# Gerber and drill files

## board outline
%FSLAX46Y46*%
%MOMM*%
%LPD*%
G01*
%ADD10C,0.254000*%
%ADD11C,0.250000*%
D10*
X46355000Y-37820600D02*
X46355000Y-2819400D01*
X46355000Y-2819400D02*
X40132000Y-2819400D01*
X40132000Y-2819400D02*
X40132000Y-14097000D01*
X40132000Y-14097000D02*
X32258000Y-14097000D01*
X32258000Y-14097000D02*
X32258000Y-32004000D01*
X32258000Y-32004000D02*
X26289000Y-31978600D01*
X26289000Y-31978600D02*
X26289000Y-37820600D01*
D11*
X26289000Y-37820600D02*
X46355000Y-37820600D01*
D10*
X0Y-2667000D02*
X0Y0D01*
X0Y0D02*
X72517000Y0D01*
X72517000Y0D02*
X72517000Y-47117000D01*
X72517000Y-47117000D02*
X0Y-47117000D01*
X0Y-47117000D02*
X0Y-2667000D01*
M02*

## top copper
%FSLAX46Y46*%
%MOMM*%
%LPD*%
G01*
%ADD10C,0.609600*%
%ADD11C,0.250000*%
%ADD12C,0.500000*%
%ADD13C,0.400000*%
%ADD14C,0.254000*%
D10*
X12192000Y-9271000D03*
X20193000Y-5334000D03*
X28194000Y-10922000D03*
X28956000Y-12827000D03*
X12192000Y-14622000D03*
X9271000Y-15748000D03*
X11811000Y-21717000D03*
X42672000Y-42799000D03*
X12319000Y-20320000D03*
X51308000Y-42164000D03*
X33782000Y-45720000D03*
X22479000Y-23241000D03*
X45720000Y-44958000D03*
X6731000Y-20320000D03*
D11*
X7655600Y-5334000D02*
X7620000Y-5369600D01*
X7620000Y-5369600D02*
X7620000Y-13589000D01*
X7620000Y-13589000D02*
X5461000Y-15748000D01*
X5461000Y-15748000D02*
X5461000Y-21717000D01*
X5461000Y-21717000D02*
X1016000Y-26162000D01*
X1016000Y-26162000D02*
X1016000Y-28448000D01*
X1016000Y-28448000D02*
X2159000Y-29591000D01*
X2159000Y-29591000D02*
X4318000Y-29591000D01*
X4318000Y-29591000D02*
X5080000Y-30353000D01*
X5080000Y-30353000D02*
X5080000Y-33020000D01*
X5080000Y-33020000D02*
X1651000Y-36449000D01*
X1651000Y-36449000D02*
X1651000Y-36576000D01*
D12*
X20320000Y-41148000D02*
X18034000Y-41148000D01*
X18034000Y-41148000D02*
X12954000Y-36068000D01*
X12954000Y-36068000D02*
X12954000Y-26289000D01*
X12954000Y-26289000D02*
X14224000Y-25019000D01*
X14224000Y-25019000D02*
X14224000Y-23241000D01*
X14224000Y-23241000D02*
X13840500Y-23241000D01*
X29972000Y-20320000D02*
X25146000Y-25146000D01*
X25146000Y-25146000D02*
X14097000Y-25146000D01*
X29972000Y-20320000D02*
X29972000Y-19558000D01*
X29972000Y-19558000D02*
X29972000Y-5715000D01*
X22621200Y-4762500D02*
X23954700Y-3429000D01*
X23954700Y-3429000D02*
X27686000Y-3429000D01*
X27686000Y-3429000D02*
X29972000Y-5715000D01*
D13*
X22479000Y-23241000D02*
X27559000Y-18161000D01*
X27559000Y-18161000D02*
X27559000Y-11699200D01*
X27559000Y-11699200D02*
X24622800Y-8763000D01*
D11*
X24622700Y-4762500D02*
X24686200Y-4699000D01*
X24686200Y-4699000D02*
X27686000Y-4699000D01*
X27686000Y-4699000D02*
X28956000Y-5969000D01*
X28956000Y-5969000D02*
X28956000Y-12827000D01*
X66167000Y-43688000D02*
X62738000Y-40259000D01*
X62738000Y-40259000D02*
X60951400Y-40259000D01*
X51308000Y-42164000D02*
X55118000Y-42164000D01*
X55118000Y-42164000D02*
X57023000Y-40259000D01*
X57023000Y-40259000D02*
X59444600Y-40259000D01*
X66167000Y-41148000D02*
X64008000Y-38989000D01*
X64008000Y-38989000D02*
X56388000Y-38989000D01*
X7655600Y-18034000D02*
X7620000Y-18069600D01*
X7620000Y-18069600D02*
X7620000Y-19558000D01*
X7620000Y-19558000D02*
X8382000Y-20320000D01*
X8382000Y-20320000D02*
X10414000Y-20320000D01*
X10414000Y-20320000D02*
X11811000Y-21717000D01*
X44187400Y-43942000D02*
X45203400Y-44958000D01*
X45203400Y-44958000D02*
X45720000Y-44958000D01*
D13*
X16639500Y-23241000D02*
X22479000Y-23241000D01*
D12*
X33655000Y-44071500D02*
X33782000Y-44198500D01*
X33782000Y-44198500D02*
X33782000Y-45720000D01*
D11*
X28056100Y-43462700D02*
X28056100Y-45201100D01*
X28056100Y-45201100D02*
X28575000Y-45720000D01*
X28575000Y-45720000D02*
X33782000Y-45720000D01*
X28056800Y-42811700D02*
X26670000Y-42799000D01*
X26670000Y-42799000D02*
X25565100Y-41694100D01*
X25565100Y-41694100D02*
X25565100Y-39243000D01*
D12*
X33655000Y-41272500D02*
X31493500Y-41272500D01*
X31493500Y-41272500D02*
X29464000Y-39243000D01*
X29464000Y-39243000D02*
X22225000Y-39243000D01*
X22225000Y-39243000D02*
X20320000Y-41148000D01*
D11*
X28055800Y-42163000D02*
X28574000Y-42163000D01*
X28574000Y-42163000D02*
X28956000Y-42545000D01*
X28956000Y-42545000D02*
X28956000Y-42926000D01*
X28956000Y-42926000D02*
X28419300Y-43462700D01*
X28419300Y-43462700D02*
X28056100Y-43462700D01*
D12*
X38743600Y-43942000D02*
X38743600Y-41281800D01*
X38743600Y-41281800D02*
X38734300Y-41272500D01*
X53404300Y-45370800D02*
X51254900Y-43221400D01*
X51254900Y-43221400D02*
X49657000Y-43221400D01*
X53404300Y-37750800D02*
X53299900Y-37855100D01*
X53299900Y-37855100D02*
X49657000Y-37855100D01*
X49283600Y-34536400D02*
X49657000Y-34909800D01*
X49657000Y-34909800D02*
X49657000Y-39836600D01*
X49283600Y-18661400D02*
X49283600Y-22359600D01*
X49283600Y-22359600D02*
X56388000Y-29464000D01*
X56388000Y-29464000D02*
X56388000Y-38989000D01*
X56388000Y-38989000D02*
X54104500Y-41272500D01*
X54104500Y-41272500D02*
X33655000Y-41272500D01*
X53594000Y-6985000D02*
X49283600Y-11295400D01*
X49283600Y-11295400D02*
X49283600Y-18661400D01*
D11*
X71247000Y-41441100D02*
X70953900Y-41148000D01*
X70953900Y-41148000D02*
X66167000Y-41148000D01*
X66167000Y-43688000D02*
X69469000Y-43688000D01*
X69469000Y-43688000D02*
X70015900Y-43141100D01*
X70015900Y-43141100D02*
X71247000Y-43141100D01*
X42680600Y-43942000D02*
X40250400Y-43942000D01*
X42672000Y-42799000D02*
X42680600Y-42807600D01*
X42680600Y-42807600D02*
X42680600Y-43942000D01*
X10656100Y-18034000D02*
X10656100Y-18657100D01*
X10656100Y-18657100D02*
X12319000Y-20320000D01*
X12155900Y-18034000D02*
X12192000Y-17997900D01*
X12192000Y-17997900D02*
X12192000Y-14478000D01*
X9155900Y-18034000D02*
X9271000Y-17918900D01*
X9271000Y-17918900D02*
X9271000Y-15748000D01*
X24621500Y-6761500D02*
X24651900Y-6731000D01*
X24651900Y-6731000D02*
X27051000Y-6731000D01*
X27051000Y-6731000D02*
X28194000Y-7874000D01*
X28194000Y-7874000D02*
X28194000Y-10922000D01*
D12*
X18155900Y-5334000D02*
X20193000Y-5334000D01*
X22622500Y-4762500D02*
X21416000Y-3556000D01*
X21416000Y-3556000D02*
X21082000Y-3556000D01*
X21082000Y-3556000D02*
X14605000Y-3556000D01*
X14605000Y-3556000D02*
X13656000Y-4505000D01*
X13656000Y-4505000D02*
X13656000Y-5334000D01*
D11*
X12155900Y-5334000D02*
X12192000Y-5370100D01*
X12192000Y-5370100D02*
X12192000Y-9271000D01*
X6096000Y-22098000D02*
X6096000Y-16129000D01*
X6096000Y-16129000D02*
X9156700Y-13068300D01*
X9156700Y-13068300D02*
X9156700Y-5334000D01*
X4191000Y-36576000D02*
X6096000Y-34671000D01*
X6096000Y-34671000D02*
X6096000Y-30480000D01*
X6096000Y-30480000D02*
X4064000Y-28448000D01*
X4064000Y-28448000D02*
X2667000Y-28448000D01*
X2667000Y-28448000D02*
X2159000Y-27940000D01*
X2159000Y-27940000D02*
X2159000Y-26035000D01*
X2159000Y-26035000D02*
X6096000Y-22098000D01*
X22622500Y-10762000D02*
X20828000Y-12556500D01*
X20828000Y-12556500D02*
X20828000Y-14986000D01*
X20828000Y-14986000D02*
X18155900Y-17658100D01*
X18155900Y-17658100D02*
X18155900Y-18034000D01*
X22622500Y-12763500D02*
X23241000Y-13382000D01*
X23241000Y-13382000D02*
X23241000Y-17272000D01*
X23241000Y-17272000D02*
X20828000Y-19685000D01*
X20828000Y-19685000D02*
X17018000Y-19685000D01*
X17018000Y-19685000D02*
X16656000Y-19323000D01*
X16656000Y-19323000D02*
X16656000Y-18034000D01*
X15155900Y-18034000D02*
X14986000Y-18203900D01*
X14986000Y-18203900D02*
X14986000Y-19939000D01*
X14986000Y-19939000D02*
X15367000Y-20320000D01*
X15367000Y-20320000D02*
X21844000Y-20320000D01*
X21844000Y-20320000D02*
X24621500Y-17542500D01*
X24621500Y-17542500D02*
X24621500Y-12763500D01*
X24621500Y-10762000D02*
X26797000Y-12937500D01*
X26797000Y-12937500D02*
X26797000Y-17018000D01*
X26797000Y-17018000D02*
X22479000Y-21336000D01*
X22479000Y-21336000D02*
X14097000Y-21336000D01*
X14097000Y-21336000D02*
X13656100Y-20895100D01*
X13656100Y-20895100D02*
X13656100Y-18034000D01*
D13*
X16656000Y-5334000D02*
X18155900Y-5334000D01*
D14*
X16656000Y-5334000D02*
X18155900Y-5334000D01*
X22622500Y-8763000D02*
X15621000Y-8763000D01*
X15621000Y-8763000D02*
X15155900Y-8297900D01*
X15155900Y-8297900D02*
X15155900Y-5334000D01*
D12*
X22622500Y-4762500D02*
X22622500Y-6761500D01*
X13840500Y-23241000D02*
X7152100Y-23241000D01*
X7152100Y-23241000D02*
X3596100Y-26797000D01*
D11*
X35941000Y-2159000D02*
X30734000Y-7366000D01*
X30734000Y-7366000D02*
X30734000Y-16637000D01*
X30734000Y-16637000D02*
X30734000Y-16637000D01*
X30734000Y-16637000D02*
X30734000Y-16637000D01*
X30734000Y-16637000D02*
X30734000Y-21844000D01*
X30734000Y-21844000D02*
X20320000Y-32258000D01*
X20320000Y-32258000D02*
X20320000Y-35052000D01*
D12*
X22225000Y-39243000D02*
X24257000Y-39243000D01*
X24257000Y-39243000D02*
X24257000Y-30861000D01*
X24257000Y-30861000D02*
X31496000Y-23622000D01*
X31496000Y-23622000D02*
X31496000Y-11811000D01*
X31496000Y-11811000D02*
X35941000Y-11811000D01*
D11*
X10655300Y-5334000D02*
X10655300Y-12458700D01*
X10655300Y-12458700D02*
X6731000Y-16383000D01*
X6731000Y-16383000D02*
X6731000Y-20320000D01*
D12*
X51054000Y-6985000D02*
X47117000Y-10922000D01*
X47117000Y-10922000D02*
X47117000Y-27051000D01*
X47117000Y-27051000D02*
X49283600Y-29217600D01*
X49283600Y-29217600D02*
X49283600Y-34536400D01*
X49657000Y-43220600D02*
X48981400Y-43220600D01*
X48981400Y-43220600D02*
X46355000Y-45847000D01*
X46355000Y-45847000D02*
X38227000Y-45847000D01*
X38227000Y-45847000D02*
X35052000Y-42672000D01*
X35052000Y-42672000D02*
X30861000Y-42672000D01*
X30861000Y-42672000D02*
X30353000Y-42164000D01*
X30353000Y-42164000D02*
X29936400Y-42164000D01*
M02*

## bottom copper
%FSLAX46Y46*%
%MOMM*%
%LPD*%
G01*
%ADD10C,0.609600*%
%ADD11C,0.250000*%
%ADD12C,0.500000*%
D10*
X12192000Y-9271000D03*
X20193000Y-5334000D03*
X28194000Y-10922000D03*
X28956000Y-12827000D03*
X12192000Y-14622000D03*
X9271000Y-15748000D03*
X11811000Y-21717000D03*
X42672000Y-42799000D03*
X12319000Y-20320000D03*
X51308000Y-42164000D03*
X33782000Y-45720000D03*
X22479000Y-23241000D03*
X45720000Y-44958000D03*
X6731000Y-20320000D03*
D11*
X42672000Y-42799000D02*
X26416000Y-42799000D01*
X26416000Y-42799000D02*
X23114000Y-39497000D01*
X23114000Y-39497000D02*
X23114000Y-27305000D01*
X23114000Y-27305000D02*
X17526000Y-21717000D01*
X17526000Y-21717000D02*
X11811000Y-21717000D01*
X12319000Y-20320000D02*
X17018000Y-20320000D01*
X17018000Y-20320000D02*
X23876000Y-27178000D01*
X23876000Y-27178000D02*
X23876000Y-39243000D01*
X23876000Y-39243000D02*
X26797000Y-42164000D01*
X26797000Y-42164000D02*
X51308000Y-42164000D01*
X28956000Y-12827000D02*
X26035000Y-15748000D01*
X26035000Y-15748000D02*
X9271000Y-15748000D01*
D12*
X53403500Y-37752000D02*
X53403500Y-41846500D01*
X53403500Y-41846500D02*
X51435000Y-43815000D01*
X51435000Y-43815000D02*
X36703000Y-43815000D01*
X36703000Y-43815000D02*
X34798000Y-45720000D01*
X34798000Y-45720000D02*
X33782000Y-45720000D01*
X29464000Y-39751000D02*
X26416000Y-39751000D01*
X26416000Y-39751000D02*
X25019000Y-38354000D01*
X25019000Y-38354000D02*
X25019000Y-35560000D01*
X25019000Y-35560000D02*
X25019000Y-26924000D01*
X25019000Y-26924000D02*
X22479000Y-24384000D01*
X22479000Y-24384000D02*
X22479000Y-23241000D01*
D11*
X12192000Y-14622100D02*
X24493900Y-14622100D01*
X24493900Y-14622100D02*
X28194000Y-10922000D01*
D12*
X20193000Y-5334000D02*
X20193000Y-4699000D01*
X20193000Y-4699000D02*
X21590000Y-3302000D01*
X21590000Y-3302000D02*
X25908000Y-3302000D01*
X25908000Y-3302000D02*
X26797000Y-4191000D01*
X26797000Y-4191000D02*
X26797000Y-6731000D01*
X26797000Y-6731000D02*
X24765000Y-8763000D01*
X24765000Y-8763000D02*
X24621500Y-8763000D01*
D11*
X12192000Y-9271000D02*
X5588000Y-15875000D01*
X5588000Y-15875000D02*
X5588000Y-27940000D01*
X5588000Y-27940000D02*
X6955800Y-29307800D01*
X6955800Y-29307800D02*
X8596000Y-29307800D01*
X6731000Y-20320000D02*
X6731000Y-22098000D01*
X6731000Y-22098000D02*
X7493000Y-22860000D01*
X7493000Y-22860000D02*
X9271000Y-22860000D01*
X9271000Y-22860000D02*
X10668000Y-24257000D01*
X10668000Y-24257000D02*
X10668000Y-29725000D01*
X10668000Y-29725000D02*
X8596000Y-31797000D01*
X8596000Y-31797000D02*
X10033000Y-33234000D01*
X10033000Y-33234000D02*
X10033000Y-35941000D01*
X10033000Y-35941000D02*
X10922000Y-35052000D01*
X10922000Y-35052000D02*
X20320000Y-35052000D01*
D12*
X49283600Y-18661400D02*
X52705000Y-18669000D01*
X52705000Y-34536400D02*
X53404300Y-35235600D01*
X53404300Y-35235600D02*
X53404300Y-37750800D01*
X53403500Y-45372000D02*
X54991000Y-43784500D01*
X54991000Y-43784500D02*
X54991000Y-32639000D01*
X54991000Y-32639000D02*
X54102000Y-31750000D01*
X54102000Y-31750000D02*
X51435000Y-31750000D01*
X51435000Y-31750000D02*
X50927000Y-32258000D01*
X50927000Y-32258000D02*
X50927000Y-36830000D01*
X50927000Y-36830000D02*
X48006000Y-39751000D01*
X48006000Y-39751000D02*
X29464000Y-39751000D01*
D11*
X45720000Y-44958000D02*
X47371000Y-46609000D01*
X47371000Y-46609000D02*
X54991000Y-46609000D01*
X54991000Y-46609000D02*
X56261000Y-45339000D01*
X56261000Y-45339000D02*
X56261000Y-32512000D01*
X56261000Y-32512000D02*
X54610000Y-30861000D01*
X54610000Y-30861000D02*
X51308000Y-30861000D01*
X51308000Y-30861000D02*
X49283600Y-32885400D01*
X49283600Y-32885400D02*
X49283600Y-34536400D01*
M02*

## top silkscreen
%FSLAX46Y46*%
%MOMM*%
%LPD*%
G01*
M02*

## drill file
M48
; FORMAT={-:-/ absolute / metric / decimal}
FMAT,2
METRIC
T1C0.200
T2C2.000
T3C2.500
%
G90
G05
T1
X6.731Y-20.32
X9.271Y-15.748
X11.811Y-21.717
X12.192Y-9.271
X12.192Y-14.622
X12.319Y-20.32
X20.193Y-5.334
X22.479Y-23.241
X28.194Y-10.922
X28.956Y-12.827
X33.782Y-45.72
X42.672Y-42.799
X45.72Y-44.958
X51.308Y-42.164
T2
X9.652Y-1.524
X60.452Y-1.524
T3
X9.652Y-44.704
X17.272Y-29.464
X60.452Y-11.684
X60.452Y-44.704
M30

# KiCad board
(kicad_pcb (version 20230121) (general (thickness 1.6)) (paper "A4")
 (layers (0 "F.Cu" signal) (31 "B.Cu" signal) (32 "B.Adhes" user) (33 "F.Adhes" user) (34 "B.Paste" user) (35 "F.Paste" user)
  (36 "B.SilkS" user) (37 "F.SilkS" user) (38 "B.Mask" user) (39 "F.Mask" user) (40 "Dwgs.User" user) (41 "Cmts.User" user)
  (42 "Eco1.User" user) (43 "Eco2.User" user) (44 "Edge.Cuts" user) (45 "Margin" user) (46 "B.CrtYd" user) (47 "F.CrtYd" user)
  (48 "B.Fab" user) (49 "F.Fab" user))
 (gr_line (start 46.3550 37.8206) (end 46.3550 2.8194) (layer "Edge.Cuts") (width 0.2540))
 (gr_line (start 46.3550 2.8194) (end 40.1320 2.8194) (layer "Edge.Cuts") (width 0.2540))
 (gr_line (start 40.1320 2.8194) (end 40.1320 14.0970) (layer "Edge.Cuts") (width 0.2540))
 (gr_line (start 40.1320 14.0970) (end 32.2580 14.0970) (layer "Edge.Cuts") (width 0.2540))
 (gr_line (start 32.2580 14.0970) (end 32.2580 32.0040) (layer "Edge.Cuts") (width 0.2540))
 (gr_line (start 32.2580 32.0040) (end 26.2890 31.9786) (layer "Edge.Cuts") (width 0.2540))
 (gr_line (start 26.2890 31.9786) (end 26.2890 37.8206) (layer "Edge.Cuts") (width 0.2540))
 (gr_line (start 26.2890 37.8206) (end 46.3550 37.8206) (layer "Edge.Cuts") (width 0.2500))
 (gr_line (start 0.0000 2.6670) (end 0.0000 0.0000) (layer "Edge.Cuts") (width 0.2540))
 (gr_line (start 0.0000 0.0000) (end 72.5170 0.0000) (layer "Edge.Cuts") (width 0.2540))
 (gr_line (start 72.5170 0.0000) (end 72.5170 47.1170) (layer "Edge.Cuts") (width 0.2540))
 (gr_line (start 72.5170 47.1170) (end 0.0000 47.1170) (layer "Edge.Cuts") (width 0.2540))
 (gr_line (start 0.0000 47.1170) (end 0.0000 2.6670) (layer "Edge.Cuts") (width 0.2540))
 (segment (start 7.6556 5.3340) (end 7.6200 5.3696) (width 0.2500) (layer "F.Cu") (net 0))
 (segment (start 7.6200 5.3696) (end 7.6200 13.5890) (width 0.2500) (layer "F.Cu") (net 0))
 (segment (start 7.6200 13.5890) (end 5.4610 15.7480) (width 0.2500) (layer "F.Cu") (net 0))
 (segment (start 5.4610 15.7480) (end 5.4610 21.7170) (width 0.2500) (layer "F.Cu") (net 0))
 (segment (start 5.4610 21.7170) (end 1.0160 26.1620) (width 0.2500) (layer "F.Cu") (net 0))
 (segment (start 1.0160 26.1620) (end 1.0160 28.4480) (width 0.2500) (layer "F.Cu") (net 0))
 (segment (start 1.0160 28.4480) (end 2.1590 29.5910) (width 0.2500) (layer "F.Cu") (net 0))
 (segment (start 2.1590 29.5910) (end 4.3180 29.5910) (width 0.2500) (layer "F.Cu") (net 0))
 (segment (start 4.3180 29.5910) (end 5.0800 30.3530) (width 0.2500) (layer "F.Cu") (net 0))
 (segment (start 5.0800 30.3530) (end 5.0800 33.0200) (width 0.2500) (layer "F.Cu") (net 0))
 (segment (start 5.0800 33.0200) (end 1.6510 36.4490) (width 0.2500) (layer "F.Cu") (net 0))
 (segment (start 1.6510 36.4490) (end 1.6510 36.5760) (width 0.2500) (layer "F.Cu") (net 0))
 (segment (start 20.3200 41.1480) (end 18.0340 41.1480) (width 0.5000) (layer "F.Cu") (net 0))
 (segment (start 18.0340 41.1480) (end 12.9540 36.0680) (width 0.5000) (layer "F.Cu") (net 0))
 (segment (start 12.9540 36.0680) (end 12.9540 26.2890) (width 0.5000) (layer "F.Cu") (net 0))
 (segment (start 12.9540 26.2890) (end 14.2240 25.0190) (width 0.5000) (layer "F.Cu") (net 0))
 (segment (start 14.2240 25.0190) (end 14.2240 23.2410) (width 0.5000) (layer "F.Cu") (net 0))
 (segment (start 14.2240 23.2410) (end 13.8405 23.2410) (width 0.5000) (layer "F.Cu") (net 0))
 (segment (start 29.9720 20.3200) (end 25.1460 25.1460) (width 0.5000) (layer "F.Cu") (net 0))
 (segment (start 25.1460 25.1460) (end 14.0970 25.1460) (width 0.5000) (layer "F.Cu") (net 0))
 (segment (start 29.9720 20.3200) (end 29.9720 19.5580) (width 0.5000) (layer "F.Cu") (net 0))
 (segment (start 29.9720 19.5580) (end 29.9720 5.7150) (width 0.5000) (layer "F.Cu") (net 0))
 (segment (start 22.6212 4.7625) (end 23.9547 3.4290) (width 0.5000) (layer "F.Cu") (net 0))
 (segment (start 23.9547 3.4290) (end 27.6860 3.4290) (width 0.5000) (layer "F.Cu") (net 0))
 (segment (start 27.6860 3.4290) (end 29.9720 5.7150) (width 0.5000) (layer "F.Cu") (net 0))
 (segment (start 22.4790 23.2410) (end 27.5590 18.1610) (width 0.4000) (layer "F.Cu") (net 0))
 (segment (start 27.5590 18.1610) (end 27.5590 11.6992) (width 0.4000) (layer "F.Cu") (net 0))
 (segment (start 27.5590 11.6992) (end 24.6228 8.7630) (width 0.4000) (layer "F.Cu") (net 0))
 (segment (start 24.6227 4.7625) (end 24.6862 4.6990) (width 0.2500) (layer "F.Cu") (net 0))
 (segment (start 24.6862 4.6990) (end 27.6860 4.6990) (width 0.2500) (layer "F.Cu") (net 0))
 (segment (start 27.6860 4.6990) (end 28.9560 5.9690) (width 0.2500) (layer "F.Cu") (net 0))
 (segment (start 28.9560 5.9690) (end 28.9560 12.8270) (width 0.2500) (layer "F.Cu") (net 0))
 (segment (start 66.1670 43.6880) (end 62.7380 40.2590) (width 0.2500) (layer "F.Cu") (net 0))
 (segment (start 62.7380 40.2590) (end 60.9514 40.2590) (width 0.2500) (layer "F.Cu") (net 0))
 (segment (start 51.3080 42.1640) (end 55.1180 42.1640) (width 0.2500) (layer "F.Cu") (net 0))
 (segment (start 55.1180 42.1640) (end 57.0230 40.2590) (width 0.2500) (layer "F.Cu") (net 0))
 (segment (start 57.0230 40.2590) (end 59.4446 40.2590) (width 0.2500) (layer "F.Cu") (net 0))
 (segment (start 66.1670 41.1480) (end 64.0080 38.9890) (width 0.2500) (layer "F.Cu") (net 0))
 (segment (start 64.0080 38.9890) (end 56.3880 38.9890) (width 0.2500) (layer "F.Cu") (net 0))
 (segment (start 7.6556 18.0340) (end 7.6200 18.0696) (width 0.2500) (layer "F.Cu") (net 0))
 (segment (start 7.6200 18.0696) (end 7.6200 19.5580) (width 0.2500) (layer "F.Cu") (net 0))
 (segment (start 7.6200 19.5580) (end 8.3820 20.3200) (width 0.2500) (layer "F.Cu") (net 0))
 (segment (start 8.3820 20.3200) (end 10.4140 20.3200) (width 0.2500) (layer "F.Cu") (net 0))
 (segment (start 10.4140 20.3200) (end 11.8110 21.7170) (width 0.2500) (layer "F.Cu") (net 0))
 (segment (start 44.1874 43.9420) (end 45.2034 44.9580) (width 0.2500) (layer "F.Cu") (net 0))
 (segment (start 45.2034 44.9580) (end 45.7200 44.9580) (width 0.2500) (layer "F.Cu") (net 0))
 (segment (start 16.6395 23.2410) (end 22.4790 23.2410) (width 0.4000) (layer "F.Cu") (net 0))
 (segment (start 33.6550 44.0715) (end 33.7820 44.1985) (width 0.5000) (layer "F.Cu") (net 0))
 (segment (start 33.7820 44.1985) (end 33.7820 45.7200) (width 0.5000) (layer "F.Cu") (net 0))
 (segment (start 28.0561 43.4627) (end 28.0561 45.2011) (width 0.2500) (layer "F.Cu") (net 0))
 (segment (start 28.0561 45.2011) (end 28.5750 45.7200) (width 0.2500) (layer "F.Cu") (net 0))
 (segment (start 28.5750 45.7200) (end 33.7820 45.7200) (width 0.2500) (layer "F.Cu") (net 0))
 (segment (start 28.0568 42.8117) (end 26.6700 42.7990) (width 0.2500) (layer "F.Cu") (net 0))
 (segment (start 26.6700 42.7990) (end 25.5651 41.6941) (width 0.2500) (layer "F.Cu") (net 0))
 (segment (start 25.5651 41.6941) (end 25.5651 39.2430) (width 0.2500) (layer "F.Cu") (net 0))
 (segment (start 33.6550 41.2725) (end 31.4935 41.2725) (width 0.5000) (layer "F.Cu") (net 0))
 (segment (start 31.4935 41.2725) (end 29.4640 39.2430) (width 0.5000) (layer "F.Cu") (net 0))
 (segment (start 29.4640 39.2430) (end 22.2250 39.2430) (width 0.5000) (layer "F.Cu") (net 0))
 (segment (start 22.2250 39.2430) (end 20.3200 41.1480) (width 0.5000) (layer "F.Cu") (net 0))
 (segment (start 28.0558 42.1630) (end 28.5740 42.1630) (width 0.2500) (layer "F.Cu") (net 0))
 (segment (start 28.5740 42.1630) (end 28.9560 42.5450) (width 0.2500) (layer "F.Cu") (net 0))
 (segment (start 28.9560 42.5450) (end 28.9560 42.9260) (width 0.2500) (layer "F.Cu") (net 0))
 (segment (start 28.9560 42.9260) (end 28.4193 43.4627) (width 0.2500) (layer "F.Cu") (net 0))
 (segment (start 28.4193 43.4627) (end 28.0561 43.4627) (width 0.2500) (layer "F.Cu") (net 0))
 (segment (start 38.7436 43.9420) (end 38.7436 41.2818) (width 0.5000) (layer "F.Cu") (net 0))
 (segment (start 38.7436 41.2818) (end 38.7343 41.2725) (width 0.5000) (layer "F.Cu") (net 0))
 (segment (start 53.4043 45.3708) (end 51.2549 43.2214) (width 0.5000) (layer "F.Cu") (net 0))
 (segment (start 51.2549 43.2214) (end 49.6570 43.2214) (width 0.5000) (layer "F.Cu") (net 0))
 (segment (start 53.4043 37.7508) (end 53.2999 37.8551) (width 0.5000) (layer "F.Cu") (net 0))
 (segment (start 53.2999 37.8551) (end 49.6570 37.8551) (width 0.5000) (layer "F.Cu") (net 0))
 (segment (start 49.2836 34.5364) (end 49.6570 34.9098) (width 0.5000) (layer "F.Cu") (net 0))
 (segment (start 49.6570 34.9098) (end 49.6570 39.8366) (width 0.5000) (layer "F.Cu") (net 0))
 (segment (start 49.2836 18.6614) (end 49.2836 22.3596) (width 0.5000) (layer "F.Cu") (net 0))
 (segment (start 49.2836 22.3596) (end 56.3880 29.4640) (width 0.5000) (layer "F.Cu") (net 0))
 (segment (start 56.3880 29.4640) (end 56.3880 38.9890) (width 0.5000) (layer "F.Cu") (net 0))
 (segment (start 56.3880 38.9890) (end 54.1045 41.2725) (width 0.5000) (layer "F.Cu") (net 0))
 (segment (start 54.1045 41.2725) (end 33.6550 41.2725) (width 0.5000) (layer "F.Cu") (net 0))
 (segment (start 53.5940 6.9850) (end 49.2836 11.2954) (width 0.5000) (layer "F.Cu") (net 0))
 (segment (start 49.2836 11.2954) (end 49.2836 18.6614) (width 0.5000) (layer "F.Cu") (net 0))
 (segment (start 71.2470 41.4411) (end 70.9539 41.1480) (width 0.2500) (layer "F.Cu") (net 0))
 (segment (start 70.9539 41.1480) (end 66.1670 41.1480) (width 0.2500) (layer "F.Cu") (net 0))
 (segment (start 66.1670 43.6880) (end 69.4690 43.6880) (width 0.2500) (layer "F.Cu") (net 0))
 (segment (start 69.4690 43.6880) (end 70.0159 43.1411) (width 0.2500) (layer "F.Cu") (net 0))
 (segment (start 70.0159 43.1411) (end 71.2470 43.1411) (width 0.2500) (layer "F.Cu") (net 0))
 (segment (start 42.6806 43.9420) (end 40.2504 43.9420) (width 0.2500) (layer "F.Cu") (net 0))
 (segment (start 42.6720 42.7990) (end 42.6806 42.8076) (width 0.2500) (layer "F.Cu") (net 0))
 (segment (start 42.6806 42.8076) (end 42.6806 43.9420) (width 0.2500) (layer "F.Cu") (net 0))
 (segment (start 10.6561 18.0340) (end 10.6561 18.6571) (width 0.2500) (layer "F.Cu") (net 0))
 (segment (start 10.6561 18.6571) (end 12.3190 20.3200) (width 0.2500) (layer "F.Cu") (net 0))
 (segment (start 12.1559 18.0340) (end 12.1920 17.9979) (width 0.2500) (layer "F.Cu") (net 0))
 (segment (start 12.1920 17.9979) (end 12.1920 14.4780) (width 0.2500) (layer "F.Cu") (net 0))
 (segment (start 9.1559 18.0340) (end 9.2710 17.9189) (width 0.2500) (layer "F.Cu") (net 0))
 (segment (start 9.2710 17.9189) (end 9.2710 15.7480) (width 0.2500) (layer "F.Cu") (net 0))
 (segment (start 24.6215 6.7615) (end 24.6519 6.7310) (width 0.2500) (layer "F.Cu") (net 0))
 (segment (start 24.6519 6.7310) (end 27.0510 6.7310) (width 0.2500) (layer "F.Cu") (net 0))
 (segment (start 27.0510 6.7310) (end 28.1940 7.8740) (width 0.2500) (layer "F.Cu") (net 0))
 (segment (start 28.1940 7.8740) (end 28.1940 10.9220) (width 0.2500) (layer "F.Cu") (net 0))
 (segment (start 18.1559 5.3340) (end 20.1930 5.3340) (width 0.5000) (layer "F.Cu") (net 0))
 (segment (start 22.6225 4.7625) (end 21.4160 3.5560) (width 0.5000) (layer "F.Cu") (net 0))
 (segment (start 21.4160 3.5560) (end 21.0820 3.5560) (width 0.5000) (layer "F.Cu") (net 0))
 (segment (start 21.0820 3.5560) (end 14.6050 3.5560) (width 0.5000) (layer "F.Cu") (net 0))
 (segment (start 14.6050 3.5560) (end 13.6560 4.5050) (width 0.5000) (layer "F.Cu") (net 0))
 (segment (start 13.6560 4.5050) (end 13.6560 5.3340) (width 0.5000) (layer "F.Cu") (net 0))
 (segment (start 12.1559 5.3340) (end 12.1920 5.3701) (width 0.2500) (layer "F.Cu") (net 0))
 (segment (start 12.1920 5.3701) (end 12.1920 9.2710) (width 0.2500) (layer "F.Cu") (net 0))
 (segment (start 6.0960 22.0980) (end 6.0960 16.1290) (width 0.2500) (layer "F.Cu") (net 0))
 (segment (start 6.0960 16.1290) (end 9.1567 13.0683) (width 0.2500) (layer "F.Cu") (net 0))
 (segment (start 9.1567 13.0683) (end 9.1567 5.3340) (width 0.2500) (layer "F.Cu") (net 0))
 (segment (start 4.1910 36.5760) (end 6.0960 34.6710) (width 0.2500) (layer "F.Cu") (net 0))
 (segment (start 6.0960 34.6710) (end 6.0960 30.4800) (width 0.2500) (layer "F.Cu") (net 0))
 (segment (start 6.0960 30.4800) (end 4.0640 28.4480) (width 0.2500) (layer "F.Cu") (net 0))
 (segment (start 4.0640 28.4480) (end 2.6670 28.4480) (width 0.2500) (layer "F.Cu") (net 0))
 (segment (start 2.6670 28.4480) (end 2.1590 27.9400) (width 0.2500) (layer "F.Cu") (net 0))
 (segment (start 2.1590 27.9400) (end 2.1590 26.0350) (width 0.2500) (layer "F.Cu") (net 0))
 (segment (start 2.1590 26.0350) (end 6.0960 22.0980) (width 0.2500) (layer "F.Cu") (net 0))
 (segment (start 22.6225 10.7620) (end 20.8280 12.5565) (width 0.2500) (layer "F.Cu") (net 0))
 (segment (start 20.8280 12.5565) (end 20.8280 14.9860) (width 0.2500) (layer "F.Cu") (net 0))
 (segment (start 20.8280 14.9860) (end 18.1559 17.6581) (width 0.2500) (layer "F.Cu") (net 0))
 (segment (start 18.1559 17.6581) (end 18.1559 18.0340) (width 0.2500) (layer "F.Cu") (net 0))
 (segment (start 22.6225 12.7635) (end 23.2410 13.3820) (width 0.2500) (layer "F.Cu") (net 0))
 (segment (start 23.2410 13.3820) (end 23.2410 17.2720) (width 0.2500) (layer "F.Cu") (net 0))
 (segment (start 23.2410 17.2720) (end 20.8280 19.6850) (width 0.2500) (layer "F.Cu") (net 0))
 (segment (start 20.8280 19.6850) (end 17.0180 19.6850) (width 0.2500) (layer "F.Cu") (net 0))
 (segment (start 17.0180 19.6850) (end 16.6560 19.3230) (width 0.2500) (layer "F.Cu") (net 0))
 (segment (start 16.6560 19.3230) (end 16.6560 18.0340) (width 0.2500) (layer "F.Cu") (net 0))
 (segment (start 15.1559 18.0340) (end 14.9860 18.2039) (width 0.2500) (layer "F.Cu") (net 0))
 (segment (start 14.9860 18.2039) (end 14.9860 19.9390) (width 0.2500) (layer "F.Cu") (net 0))
 (segment (start 14.9860 19.9390) (end 15.3670 20.3200) (width 0.2500) (layer "F.Cu") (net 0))
 (segment (start 15.3670 20.3200) (end 21.8440 20.3200) (width 0.2500) (layer "F.Cu") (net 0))
 (segment (start 21.8440 20.3200) (end 24.6215 17.5425) (width 0.2500) (layer "F.Cu") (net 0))
 (segment (start 24.6215 17.5425) (end 24.6215 12.7635) (width 0.2500) (layer "F.Cu") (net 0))
 (segment (start 24.6215 10.7620) (end 26.7970 12.9375) (width 0.2500) (layer "F.Cu") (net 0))
 (segment (start 26.7970 12.9375) (end 26.7970 17.0180) (width 0.2500) (layer "F.Cu") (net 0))
 (segment (start 26.7970 17.0180) (end 22.4790 21.3360) (width 0.2500) (layer "F.Cu") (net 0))
 (segment (start 22.4790 21.3360) (end 14.0970 21.3360) (width 0.2500) (layer "F.Cu") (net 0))
 (segment (start 14.0970 21.3360) (end 13.6561 20.8951) (width 0.2500) (layer "F.Cu") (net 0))
 (segment (start 13.6561 20.8951) (end 13.6561 18.0340) (width 0.2500) (layer "F.Cu") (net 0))
 (segment (start 16.6560 5.3340) (end 18.1559 5.3340) (width 0.4000) (layer "F.Cu") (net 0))
 (segment (start 16.6560 5.3340) (end 18.1559 5.3340) (width 0.2540) (layer "F.Cu") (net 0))
 (segment (start 22.6225 8.7630) (end 15.6210 8.7630) (width 0.2540) (layer "F.Cu") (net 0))
 (segment (start 15.6210 8.7630) (end 15.1559 8.2979) (width 0.2540) (layer "F.Cu") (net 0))
 (segment (start 15.1559 8.2979) (end 15.1559 5.3340) (width 0.2540) (layer "F.Cu") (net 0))
 (segment (start 22.6225 4.7625) (end 22.6225 6.7615) (width 0.5000) (layer "F.Cu") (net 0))
 (segment (start 13.8405 23.2410) (end 7.1521 23.2410) (width 0.5000) (layer "F.Cu") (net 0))
 (segment (start 7.1521 23.2410) (end 3.5961 26.7970) (width 0.5000) (layer "F.Cu") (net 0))
 (segment (start 35.9410 2.1590) (end 30.7340 7.3660) (width 0.2500) (layer "F.Cu") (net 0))
 (segment (start 30.7340 7.3660) (end 30.7340 16.6370) (width 0.2500) (layer "F.Cu") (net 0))
 (segment (start 30.7340 16.6370) (end 30.7340 16.6370) (width 0.2500) (layer "F.Cu") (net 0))
 (segment (start 30.7340 16.6370) (end 30.7340 16.6370) (width 0.2500) (layer "F.Cu") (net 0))
 (segment (start 30.7340 16.6370) (end 30.7340 21.8440) (width 0.2500) (layer "F.Cu") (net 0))
 (segment (start 30.7340 21.8440) (end 20.3200 32.2580) (width 0.2500) (layer "F.Cu") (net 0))
 (segment (start 20.3200 32.2580) (end 20.3200 35.0520) (width 0.2500) (layer "F.Cu") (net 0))
 (segment (start 22.2250 39.2430) (end 24.2570 39.2430) (width 0.5000) (layer "F.Cu") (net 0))
 (segment (start 24.2570 39.2430) (end 24.2570 30.8610) (width 0.5000) (layer "F.Cu") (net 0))
 (segment (start 24.2570 30.8610) (end 31.4960 23.6220) (width 0.5000) (layer "F.Cu") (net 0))
 (segment (start 31.4960 23.6220) (end 31.4960 11.8110) (width 0.5000) (layer "F.Cu") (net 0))
 (segment (start 31.4960 11.8110) (end 35.9410 11.8110) (width 0.5000) (layer "F.Cu") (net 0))
 (segment (start 10.6553 5.3340) (end 10.6553 12.4587) (width 0.2500) (layer "F.Cu") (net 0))
 (segment (start 10.6553 12.4587) (end 6.7310 16.3830) (width 0.2500) (layer "F.Cu") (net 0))
 (segment (start 6.7310 16.3830) (end 6.7310 20.3200) (width 0.2500) (layer "F.Cu") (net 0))
 (segment (start 51.0540 6.9850) (end 47.1170 10.9220) (width 0.5000) (layer "F.Cu") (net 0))
 (segment (start 47.1170 10.9220) (end 47.1170 27.0510) (width 0.5000) (layer "F.Cu") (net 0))
 (segment (start 47.1170 27.0510) (end 49.2836 29.2176) (width 0.5000) (layer "F.Cu") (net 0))
 (segment (start 49.2836 29.2176) (end 49.2836 34.5364) (width 0.5000) (layer "F.Cu") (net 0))
 (segment (start 49.6570 43.2206) (end 48.9814 43.2206) (width 0.5000) (layer "F.Cu") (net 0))
 (segment (start 48.9814 43.2206) (end 46.3550 45.8470) (width 0.5000) (layer "F.Cu") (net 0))
 (segment (start 46.3550 45.8470) (end 38.2270 45.8470) (width 0.5000) (layer "F.Cu") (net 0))
 (segment (start 38.2270 45.8470) (end 35.0520 42.6720) (width 0.5000) (layer "F.Cu") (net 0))
 (segment (start 35.0520 42.6720) (end 30.8610 42.6720) (width 0.5000) (layer "F.Cu") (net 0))
 (segment (start 30.8610 42.6720) (end 30.3530 42.1640) (width 0.5000) (layer "F.Cu") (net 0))
 (segment (start 30.3530 42.1640) (end 29.9364 42.1640) (width 0.5000) (layer "F.Cu") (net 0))
 (segment (start 42.6720 42.7990) (end 26.4160 42.7990) (width 0.2500) (layer "B.Cu") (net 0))
 (segment (start 26.4160 42.7990) (end 23.1140 39.4970) (width 0.2500) (layer "B.Cu") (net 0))
 (segment (start 23.1140 39.4970) (end 23.1140 27.3050) (width 0.2500) (layer "B.Cu") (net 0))
 (segment (start 23.1140 27.3050) (end 17.5260 21.7170) (width 0.2500) (layer "B.Cu") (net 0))
 (segment (start 17.5260 21.7170) (end 11.8110 21.7170) (width 0.2500) (layer "B.Cu") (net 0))
 (segment (start 12.3190 20.3200) (end 17.0180 20.3200) (width 0.2500) (layer "B.Cu") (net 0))
 (segment (start 17.0180 20.3200) (end 23.8760 27.1780) (width 0.2500) (layer "B.Cu") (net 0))
 (segment (start 23.8760 27.1780) (end 23.8760 39.2430) (width 0.2500) (layer "B.Cu") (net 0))
 (segment (start 23.8760 39.2430) (end 26.7970 42.1640) (width 0.2500) (layer "B.Cu") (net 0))
 (segment (start 26.7970 42.1640) (end 51.3080 42.1640) (width 0.2500) (layer "B.Cu") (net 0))
 (segment (start 28.9560 12.8270) (end 26.0350 15.7480) (width 0.2500) (layer "B.Cu") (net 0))
 (segment (start 26.0350 15.7480) (end 9.2710 15.7480) (width 0.2500) (layer "B.Cu") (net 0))
 (segment (start 53.4035 37.7520) (end 53.4035 41.8465) (width 0.5000) (layer "B.Cu") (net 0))
 (segment (start 53.4035 41.8465) (end 51.4350 43.8150) (width 0.5000) (layer "B.Cu") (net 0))
 (segment (start 51.4350 43.8150) (end 36.7030 43.8150) (width 0.5000) (layer "B.Cu") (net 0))
 (segment (start 36.7030 43.8150) (end 34.7980 45.7200) (width 0.5000) (layer "B.Cu") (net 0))
 (segment (start 34.7980 45.7200) (end 33.7820 45.7200) (width 0.5000) (layer "B.Cu") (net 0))
 (segment (start 29.4640 39.7510) (end 26.4160 39.7510) (width 0.5000) (layer "B.Cu") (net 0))
 (segment (start 26.4160 39.7510) (end 25.0190 38.3540) (width 0.5000) (layer "B.Cu") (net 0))
 (segment (start 25.0190 38.3540) (end 25.0190 35.5600) (width 0.5000) (layer "B.Cu") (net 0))
 (segment (start 25.0190 35.5600) (end 25.0190 26.9240) (width 0.5000) (layer "B.Cu") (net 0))
 (segment (start 25.0190 26.9240) (end 22.4790 24.3840) (width 0.5000) (layer "B.Cu") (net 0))
 (segment (start 22.4790 24.3840) (end 22.4790 23.2410) (width 0.5000) (layer "B.Cu") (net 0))
 (segment (start 12.1920 14.6221) (end 24.4939 14.6221) (width 0.2500) (layer "B.Cu") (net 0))
 (segment (start 24.4939 14.6221) (end 28.1940 10.9220) (width 0.2500) (layer "B.Cu") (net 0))
 (segment (start 20.1930 5.3340) (end 20.1930 4.6990) (width 0.5000) (layer "B.Cu") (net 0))
 (segment (start 20.1930 4.6990) (end 21.5900 3.3020) (width 0.5000) (layer "B.Cu") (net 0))
 (segment (start 21.5900 3.3020) (end 25.9080 3.3020) (width 0.5000) (layer "B.Cu") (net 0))
 (segment (start 25.9080 3.3020) (end 26.7970 4.1910) (width 0.5000) (layer "B.Cu") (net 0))
 (segment (start 26.7970 4.1910) (end 26.7970 6.7310) (width 0.5000) (layer "B.Cu") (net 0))
 (segment (start 26.7970 6.7310) (end 24.7650 8.7630) (width 0.5000) (layer "B.Cu") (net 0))
 (segment (start 24.7650 8.7630) (end 24.6215 8.7630) (width 0.5000) (layer "B.Cu") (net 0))
 (segment (start 12.1920 9.2710) (end 5.5880 15.8750) (width 0.2500) (layer "B.Cu") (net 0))
 (segment (start 5.5880 15.8750) (end 5.5880 27.9400) (width 0.2500) (layer "B.Cu") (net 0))
 (segment (start 5.5880 27.9400) (end 6.9558 29.3078) (width 0.2500) (layer "B.Cu") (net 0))
 (segment (start 6.9558 29.3078) (end 8.5960 29.3078) (width 0.2500) (layer "B.Cu") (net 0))
 (segment (start 6.7310 20.3200) (end 6.7310 22.0980) (width 0.2500) (layer "B.Cu") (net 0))
 (segment (start 6.7310 22.0980) (end 7.4930 22.8600) (width 0.2500) (layer "B.Cu") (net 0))
 (segment (start 7.4930 22.8600) (end 9.2710 22.8600) (width 0.2500) (layer "B.Cu") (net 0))
 (segment (start 9.2710 22.8600) (end 10.6680 24.2570) (width 0.2500) (layer "B.Cu") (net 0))
 (segment (start 10.6680 24.2570) (end 10.6680 29.7250) (width 0.2500) (layer "B.Cu") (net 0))
 (segment (start 10.6680 29.7250) (end 8.5960 31.7970) (width 0.2500) (layer "B.Cu") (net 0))
 (segment (start 8.5960 31.7970) (end 10.0330 33.2340) (width 0.2500) (layer "B.Cu") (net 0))
 (segment (start 10.0330 33.2340) (end 10.0330 35.9410) (width 0.2500) (layer "B.Cu") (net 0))
 (segment (start 10.0330 35.9410) (end 10.9220 35.0520) (width 0.2500) (layer "B.Cu") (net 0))
 (segment (start 10.9220 35.0520) (end 20.3200 35.0520) (width 0.2500) (layer "B.Cu") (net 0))
 (segment (start 49.2836 18.6614) (end 52.7050 18.6690) (width 0.5000) (layer "B.Cu") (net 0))
 (segment (start 52.7050 34.5364) (end 53.4043 35.2356) (width 0.5000) (layer "B.Cu") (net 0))
 (segment (start 53.4043 35.2356) (end 53.4043 37.7508) (width 0.5000) (layer "B.Cu") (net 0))
 (segment (start 53.4035 45.3720) (end 54.9910 43.7845) (width 0.5000) (layer "B.Cu") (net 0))
 (segment (start 54.9910 43.7845) (end 54.9910 32.6390) (width 0.5000) (layer "B.Cu") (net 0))
 (segment (start 54.9910 32.6390) (end 54.1020 31.7500) (width 0.5000) (layer "B.Cu") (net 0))
 (segment (start 54.1020 31.7500) (end 51.4350 31.7500) (width 0.5000) (layer "B.Cu") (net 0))
 (segment (start 51.4350 31.7500) (end 50.9270 32.2580) (width 0.5000) (layer "B.Cu") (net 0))
 (segment (start 50.9270 32.2580) (end 50.9270 36.8300) (width 0.5000) (layer "B.Cu") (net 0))
 (segment (start 50.9270 36.8300) (end 48.0060 39.7510) (width 0.5000) (layer "B.Cu") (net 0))
 (segment (start 48.0060 39.7510) (end 29.4640 39.7510) (width 0.5000) (layer "B.Cu") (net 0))
 (segment (start 45.7200 44.9580) (end 47.3710 46.6090) (width 0.2500) (layer "B.Cu") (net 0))
 (segment (start 47.3710 46.6090) (end 54.9910 46.6090) (width 0.2500) (layer "B.Cu") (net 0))
 (segment (start 54.9910 46.6090) (end 56.2610 45.3390) (width 0.2500) (layer "B.Cu") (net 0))
 (segment (start 56.2610 45.3390) (end 56.2610 32.5120) (width 0.2500) (layer "B.Cu") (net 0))
 (segment (start 56.2610 32.5120) (end 54.6100 30.8610) (width 0.2500) (layer "B.Cu") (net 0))
 (segment (start 54.6100 30.8610) (end 51.3080 30.8610) (width 0.2500) (layer "B.Cu") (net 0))
 (segment (start 51.3080 30.8610) (end 49.2836 32.8854) (width 0.2500) (layer "B.Cu") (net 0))
 (segment (start 49.2836 32.8854) (end 49.2836 34.5364) (width 0.2500) (layer "B.Cu") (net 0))
 (via (at 12.1920 9.2710) (size 0.6096) (drill 0.2000) (layers "F.Cu" "B.Cu") (free) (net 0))
 (via (at 20.1930 5.3340) (size 0.6096) (drill 0.2000) (layers "F.Cu" "B.Cu") (free) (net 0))
 (via (at 28.1940 10.9220) (size 0.6096) (drill 0.2000) (layers "F.Cu" "B.Cu") (free) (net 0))
 (via (at 28.9560 12.8270) (size 0.6096) (drill 0.2000) (layers "F.Cu" "B.Cu") (free) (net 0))
 (via (at 12.1920 14.6220) (size 0.6096) (drill 0.2000) (layers "F.Cu" "B.Cu") (free) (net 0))
 (via (at 9.2710 15.7480) (size 0.6096) (drill 0.2000) (layers "F.Cu" "B.Cu") (free) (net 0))
 (via (at 11.8110 21.7170) (size 0.6096) (drill 0.2000) (layers "F.Cu" "B.Cu") (free) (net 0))
 (via (at 42.6720 42.7990) (size 0.6096) (drill 0.2000) (layers "F.Cu" "B.Cu") (free) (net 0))
 (via (at 12.3190 20.3200) (size 0.6096) (drill 0.2000) (layers "F.Cu" "B.Cu") (free) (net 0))
 (via (at 51.3080 42.1640) (size 0.6096) (drill 0.2000) (layers "F.Cu" "B.Cu") (free) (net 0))
 (via (at 33.7820 45.7200) (size 0.6096) (drill 0.2000) (layers "F.Cu" "B.Cu") (free) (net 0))
 (via (at 22.4790 23.2410) (size 0.6096) (drill 0.2000) (layers "F.Cu" "B.Cu") (free) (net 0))
 (via (at 45.7200 44.9580) (size 0.6096) (drill 0.2000) (layers "F.Cu" "B.Cu") (free) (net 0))
 (via (at 6.7310 20.3200) (size 0.6096) (drill 0.2000) (layers "F.Cu" "B.Cu") (free) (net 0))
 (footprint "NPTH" (layer "F.Cu") (at 60.4520 11.6840)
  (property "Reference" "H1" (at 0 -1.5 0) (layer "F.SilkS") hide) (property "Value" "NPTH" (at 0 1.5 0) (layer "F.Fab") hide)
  (pad "" np_thru_hole circle (at 0 0) (size 2.5000 2.5000) (drill 2.5000) (layers *.Cu *.Mask)))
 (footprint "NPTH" (layer "F.Cu") (at 9.6520 44.7040)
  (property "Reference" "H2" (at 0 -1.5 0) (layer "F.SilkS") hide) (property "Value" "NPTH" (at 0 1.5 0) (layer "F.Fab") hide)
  (pad "" np_thru_hole circle (at 0 0) (size 2.5000 2.5000) (drill 2.5000) (layers *.Cu *.Mask)))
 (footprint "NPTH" (layer "F.Cu") (at 60.4520 44.7040)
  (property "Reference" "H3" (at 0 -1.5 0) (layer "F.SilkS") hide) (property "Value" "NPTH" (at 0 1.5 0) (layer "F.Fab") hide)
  (pad "" np_thru_hole circle (at 0 0) (size 2.5000 2.5000) (drill 2.5000) (layers *.Cu *.Mask)))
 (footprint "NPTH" (layer "F.Cu") (at 17.2720 29.4640)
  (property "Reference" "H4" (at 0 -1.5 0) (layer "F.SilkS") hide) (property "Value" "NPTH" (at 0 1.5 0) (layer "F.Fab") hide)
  (pad "" np_thru_hole circle (at 0 0) (size 2.5000 2.5000) (drill 2.5000) (layers *.Cu *.Mask)))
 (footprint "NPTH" (layer "F.Cu") (at 9.6520 1.5240)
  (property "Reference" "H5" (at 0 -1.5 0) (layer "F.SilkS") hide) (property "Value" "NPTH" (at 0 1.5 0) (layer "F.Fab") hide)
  (pad "" np_thru_hole circle (at 0 0) (size 2.0000 2.0000) (drill 2.0000) (layers *.Cu *.Mask)))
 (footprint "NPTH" (layer "F.Cu") (at 60.4520 1.5240)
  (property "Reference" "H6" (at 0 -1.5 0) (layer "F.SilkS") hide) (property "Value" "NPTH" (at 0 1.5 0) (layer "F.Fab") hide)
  (pad "" np_thru_hole circle (at 0 0) (size 2.0000 2.0000) (drill 2.0000) (layers *.Cu *.Mask))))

